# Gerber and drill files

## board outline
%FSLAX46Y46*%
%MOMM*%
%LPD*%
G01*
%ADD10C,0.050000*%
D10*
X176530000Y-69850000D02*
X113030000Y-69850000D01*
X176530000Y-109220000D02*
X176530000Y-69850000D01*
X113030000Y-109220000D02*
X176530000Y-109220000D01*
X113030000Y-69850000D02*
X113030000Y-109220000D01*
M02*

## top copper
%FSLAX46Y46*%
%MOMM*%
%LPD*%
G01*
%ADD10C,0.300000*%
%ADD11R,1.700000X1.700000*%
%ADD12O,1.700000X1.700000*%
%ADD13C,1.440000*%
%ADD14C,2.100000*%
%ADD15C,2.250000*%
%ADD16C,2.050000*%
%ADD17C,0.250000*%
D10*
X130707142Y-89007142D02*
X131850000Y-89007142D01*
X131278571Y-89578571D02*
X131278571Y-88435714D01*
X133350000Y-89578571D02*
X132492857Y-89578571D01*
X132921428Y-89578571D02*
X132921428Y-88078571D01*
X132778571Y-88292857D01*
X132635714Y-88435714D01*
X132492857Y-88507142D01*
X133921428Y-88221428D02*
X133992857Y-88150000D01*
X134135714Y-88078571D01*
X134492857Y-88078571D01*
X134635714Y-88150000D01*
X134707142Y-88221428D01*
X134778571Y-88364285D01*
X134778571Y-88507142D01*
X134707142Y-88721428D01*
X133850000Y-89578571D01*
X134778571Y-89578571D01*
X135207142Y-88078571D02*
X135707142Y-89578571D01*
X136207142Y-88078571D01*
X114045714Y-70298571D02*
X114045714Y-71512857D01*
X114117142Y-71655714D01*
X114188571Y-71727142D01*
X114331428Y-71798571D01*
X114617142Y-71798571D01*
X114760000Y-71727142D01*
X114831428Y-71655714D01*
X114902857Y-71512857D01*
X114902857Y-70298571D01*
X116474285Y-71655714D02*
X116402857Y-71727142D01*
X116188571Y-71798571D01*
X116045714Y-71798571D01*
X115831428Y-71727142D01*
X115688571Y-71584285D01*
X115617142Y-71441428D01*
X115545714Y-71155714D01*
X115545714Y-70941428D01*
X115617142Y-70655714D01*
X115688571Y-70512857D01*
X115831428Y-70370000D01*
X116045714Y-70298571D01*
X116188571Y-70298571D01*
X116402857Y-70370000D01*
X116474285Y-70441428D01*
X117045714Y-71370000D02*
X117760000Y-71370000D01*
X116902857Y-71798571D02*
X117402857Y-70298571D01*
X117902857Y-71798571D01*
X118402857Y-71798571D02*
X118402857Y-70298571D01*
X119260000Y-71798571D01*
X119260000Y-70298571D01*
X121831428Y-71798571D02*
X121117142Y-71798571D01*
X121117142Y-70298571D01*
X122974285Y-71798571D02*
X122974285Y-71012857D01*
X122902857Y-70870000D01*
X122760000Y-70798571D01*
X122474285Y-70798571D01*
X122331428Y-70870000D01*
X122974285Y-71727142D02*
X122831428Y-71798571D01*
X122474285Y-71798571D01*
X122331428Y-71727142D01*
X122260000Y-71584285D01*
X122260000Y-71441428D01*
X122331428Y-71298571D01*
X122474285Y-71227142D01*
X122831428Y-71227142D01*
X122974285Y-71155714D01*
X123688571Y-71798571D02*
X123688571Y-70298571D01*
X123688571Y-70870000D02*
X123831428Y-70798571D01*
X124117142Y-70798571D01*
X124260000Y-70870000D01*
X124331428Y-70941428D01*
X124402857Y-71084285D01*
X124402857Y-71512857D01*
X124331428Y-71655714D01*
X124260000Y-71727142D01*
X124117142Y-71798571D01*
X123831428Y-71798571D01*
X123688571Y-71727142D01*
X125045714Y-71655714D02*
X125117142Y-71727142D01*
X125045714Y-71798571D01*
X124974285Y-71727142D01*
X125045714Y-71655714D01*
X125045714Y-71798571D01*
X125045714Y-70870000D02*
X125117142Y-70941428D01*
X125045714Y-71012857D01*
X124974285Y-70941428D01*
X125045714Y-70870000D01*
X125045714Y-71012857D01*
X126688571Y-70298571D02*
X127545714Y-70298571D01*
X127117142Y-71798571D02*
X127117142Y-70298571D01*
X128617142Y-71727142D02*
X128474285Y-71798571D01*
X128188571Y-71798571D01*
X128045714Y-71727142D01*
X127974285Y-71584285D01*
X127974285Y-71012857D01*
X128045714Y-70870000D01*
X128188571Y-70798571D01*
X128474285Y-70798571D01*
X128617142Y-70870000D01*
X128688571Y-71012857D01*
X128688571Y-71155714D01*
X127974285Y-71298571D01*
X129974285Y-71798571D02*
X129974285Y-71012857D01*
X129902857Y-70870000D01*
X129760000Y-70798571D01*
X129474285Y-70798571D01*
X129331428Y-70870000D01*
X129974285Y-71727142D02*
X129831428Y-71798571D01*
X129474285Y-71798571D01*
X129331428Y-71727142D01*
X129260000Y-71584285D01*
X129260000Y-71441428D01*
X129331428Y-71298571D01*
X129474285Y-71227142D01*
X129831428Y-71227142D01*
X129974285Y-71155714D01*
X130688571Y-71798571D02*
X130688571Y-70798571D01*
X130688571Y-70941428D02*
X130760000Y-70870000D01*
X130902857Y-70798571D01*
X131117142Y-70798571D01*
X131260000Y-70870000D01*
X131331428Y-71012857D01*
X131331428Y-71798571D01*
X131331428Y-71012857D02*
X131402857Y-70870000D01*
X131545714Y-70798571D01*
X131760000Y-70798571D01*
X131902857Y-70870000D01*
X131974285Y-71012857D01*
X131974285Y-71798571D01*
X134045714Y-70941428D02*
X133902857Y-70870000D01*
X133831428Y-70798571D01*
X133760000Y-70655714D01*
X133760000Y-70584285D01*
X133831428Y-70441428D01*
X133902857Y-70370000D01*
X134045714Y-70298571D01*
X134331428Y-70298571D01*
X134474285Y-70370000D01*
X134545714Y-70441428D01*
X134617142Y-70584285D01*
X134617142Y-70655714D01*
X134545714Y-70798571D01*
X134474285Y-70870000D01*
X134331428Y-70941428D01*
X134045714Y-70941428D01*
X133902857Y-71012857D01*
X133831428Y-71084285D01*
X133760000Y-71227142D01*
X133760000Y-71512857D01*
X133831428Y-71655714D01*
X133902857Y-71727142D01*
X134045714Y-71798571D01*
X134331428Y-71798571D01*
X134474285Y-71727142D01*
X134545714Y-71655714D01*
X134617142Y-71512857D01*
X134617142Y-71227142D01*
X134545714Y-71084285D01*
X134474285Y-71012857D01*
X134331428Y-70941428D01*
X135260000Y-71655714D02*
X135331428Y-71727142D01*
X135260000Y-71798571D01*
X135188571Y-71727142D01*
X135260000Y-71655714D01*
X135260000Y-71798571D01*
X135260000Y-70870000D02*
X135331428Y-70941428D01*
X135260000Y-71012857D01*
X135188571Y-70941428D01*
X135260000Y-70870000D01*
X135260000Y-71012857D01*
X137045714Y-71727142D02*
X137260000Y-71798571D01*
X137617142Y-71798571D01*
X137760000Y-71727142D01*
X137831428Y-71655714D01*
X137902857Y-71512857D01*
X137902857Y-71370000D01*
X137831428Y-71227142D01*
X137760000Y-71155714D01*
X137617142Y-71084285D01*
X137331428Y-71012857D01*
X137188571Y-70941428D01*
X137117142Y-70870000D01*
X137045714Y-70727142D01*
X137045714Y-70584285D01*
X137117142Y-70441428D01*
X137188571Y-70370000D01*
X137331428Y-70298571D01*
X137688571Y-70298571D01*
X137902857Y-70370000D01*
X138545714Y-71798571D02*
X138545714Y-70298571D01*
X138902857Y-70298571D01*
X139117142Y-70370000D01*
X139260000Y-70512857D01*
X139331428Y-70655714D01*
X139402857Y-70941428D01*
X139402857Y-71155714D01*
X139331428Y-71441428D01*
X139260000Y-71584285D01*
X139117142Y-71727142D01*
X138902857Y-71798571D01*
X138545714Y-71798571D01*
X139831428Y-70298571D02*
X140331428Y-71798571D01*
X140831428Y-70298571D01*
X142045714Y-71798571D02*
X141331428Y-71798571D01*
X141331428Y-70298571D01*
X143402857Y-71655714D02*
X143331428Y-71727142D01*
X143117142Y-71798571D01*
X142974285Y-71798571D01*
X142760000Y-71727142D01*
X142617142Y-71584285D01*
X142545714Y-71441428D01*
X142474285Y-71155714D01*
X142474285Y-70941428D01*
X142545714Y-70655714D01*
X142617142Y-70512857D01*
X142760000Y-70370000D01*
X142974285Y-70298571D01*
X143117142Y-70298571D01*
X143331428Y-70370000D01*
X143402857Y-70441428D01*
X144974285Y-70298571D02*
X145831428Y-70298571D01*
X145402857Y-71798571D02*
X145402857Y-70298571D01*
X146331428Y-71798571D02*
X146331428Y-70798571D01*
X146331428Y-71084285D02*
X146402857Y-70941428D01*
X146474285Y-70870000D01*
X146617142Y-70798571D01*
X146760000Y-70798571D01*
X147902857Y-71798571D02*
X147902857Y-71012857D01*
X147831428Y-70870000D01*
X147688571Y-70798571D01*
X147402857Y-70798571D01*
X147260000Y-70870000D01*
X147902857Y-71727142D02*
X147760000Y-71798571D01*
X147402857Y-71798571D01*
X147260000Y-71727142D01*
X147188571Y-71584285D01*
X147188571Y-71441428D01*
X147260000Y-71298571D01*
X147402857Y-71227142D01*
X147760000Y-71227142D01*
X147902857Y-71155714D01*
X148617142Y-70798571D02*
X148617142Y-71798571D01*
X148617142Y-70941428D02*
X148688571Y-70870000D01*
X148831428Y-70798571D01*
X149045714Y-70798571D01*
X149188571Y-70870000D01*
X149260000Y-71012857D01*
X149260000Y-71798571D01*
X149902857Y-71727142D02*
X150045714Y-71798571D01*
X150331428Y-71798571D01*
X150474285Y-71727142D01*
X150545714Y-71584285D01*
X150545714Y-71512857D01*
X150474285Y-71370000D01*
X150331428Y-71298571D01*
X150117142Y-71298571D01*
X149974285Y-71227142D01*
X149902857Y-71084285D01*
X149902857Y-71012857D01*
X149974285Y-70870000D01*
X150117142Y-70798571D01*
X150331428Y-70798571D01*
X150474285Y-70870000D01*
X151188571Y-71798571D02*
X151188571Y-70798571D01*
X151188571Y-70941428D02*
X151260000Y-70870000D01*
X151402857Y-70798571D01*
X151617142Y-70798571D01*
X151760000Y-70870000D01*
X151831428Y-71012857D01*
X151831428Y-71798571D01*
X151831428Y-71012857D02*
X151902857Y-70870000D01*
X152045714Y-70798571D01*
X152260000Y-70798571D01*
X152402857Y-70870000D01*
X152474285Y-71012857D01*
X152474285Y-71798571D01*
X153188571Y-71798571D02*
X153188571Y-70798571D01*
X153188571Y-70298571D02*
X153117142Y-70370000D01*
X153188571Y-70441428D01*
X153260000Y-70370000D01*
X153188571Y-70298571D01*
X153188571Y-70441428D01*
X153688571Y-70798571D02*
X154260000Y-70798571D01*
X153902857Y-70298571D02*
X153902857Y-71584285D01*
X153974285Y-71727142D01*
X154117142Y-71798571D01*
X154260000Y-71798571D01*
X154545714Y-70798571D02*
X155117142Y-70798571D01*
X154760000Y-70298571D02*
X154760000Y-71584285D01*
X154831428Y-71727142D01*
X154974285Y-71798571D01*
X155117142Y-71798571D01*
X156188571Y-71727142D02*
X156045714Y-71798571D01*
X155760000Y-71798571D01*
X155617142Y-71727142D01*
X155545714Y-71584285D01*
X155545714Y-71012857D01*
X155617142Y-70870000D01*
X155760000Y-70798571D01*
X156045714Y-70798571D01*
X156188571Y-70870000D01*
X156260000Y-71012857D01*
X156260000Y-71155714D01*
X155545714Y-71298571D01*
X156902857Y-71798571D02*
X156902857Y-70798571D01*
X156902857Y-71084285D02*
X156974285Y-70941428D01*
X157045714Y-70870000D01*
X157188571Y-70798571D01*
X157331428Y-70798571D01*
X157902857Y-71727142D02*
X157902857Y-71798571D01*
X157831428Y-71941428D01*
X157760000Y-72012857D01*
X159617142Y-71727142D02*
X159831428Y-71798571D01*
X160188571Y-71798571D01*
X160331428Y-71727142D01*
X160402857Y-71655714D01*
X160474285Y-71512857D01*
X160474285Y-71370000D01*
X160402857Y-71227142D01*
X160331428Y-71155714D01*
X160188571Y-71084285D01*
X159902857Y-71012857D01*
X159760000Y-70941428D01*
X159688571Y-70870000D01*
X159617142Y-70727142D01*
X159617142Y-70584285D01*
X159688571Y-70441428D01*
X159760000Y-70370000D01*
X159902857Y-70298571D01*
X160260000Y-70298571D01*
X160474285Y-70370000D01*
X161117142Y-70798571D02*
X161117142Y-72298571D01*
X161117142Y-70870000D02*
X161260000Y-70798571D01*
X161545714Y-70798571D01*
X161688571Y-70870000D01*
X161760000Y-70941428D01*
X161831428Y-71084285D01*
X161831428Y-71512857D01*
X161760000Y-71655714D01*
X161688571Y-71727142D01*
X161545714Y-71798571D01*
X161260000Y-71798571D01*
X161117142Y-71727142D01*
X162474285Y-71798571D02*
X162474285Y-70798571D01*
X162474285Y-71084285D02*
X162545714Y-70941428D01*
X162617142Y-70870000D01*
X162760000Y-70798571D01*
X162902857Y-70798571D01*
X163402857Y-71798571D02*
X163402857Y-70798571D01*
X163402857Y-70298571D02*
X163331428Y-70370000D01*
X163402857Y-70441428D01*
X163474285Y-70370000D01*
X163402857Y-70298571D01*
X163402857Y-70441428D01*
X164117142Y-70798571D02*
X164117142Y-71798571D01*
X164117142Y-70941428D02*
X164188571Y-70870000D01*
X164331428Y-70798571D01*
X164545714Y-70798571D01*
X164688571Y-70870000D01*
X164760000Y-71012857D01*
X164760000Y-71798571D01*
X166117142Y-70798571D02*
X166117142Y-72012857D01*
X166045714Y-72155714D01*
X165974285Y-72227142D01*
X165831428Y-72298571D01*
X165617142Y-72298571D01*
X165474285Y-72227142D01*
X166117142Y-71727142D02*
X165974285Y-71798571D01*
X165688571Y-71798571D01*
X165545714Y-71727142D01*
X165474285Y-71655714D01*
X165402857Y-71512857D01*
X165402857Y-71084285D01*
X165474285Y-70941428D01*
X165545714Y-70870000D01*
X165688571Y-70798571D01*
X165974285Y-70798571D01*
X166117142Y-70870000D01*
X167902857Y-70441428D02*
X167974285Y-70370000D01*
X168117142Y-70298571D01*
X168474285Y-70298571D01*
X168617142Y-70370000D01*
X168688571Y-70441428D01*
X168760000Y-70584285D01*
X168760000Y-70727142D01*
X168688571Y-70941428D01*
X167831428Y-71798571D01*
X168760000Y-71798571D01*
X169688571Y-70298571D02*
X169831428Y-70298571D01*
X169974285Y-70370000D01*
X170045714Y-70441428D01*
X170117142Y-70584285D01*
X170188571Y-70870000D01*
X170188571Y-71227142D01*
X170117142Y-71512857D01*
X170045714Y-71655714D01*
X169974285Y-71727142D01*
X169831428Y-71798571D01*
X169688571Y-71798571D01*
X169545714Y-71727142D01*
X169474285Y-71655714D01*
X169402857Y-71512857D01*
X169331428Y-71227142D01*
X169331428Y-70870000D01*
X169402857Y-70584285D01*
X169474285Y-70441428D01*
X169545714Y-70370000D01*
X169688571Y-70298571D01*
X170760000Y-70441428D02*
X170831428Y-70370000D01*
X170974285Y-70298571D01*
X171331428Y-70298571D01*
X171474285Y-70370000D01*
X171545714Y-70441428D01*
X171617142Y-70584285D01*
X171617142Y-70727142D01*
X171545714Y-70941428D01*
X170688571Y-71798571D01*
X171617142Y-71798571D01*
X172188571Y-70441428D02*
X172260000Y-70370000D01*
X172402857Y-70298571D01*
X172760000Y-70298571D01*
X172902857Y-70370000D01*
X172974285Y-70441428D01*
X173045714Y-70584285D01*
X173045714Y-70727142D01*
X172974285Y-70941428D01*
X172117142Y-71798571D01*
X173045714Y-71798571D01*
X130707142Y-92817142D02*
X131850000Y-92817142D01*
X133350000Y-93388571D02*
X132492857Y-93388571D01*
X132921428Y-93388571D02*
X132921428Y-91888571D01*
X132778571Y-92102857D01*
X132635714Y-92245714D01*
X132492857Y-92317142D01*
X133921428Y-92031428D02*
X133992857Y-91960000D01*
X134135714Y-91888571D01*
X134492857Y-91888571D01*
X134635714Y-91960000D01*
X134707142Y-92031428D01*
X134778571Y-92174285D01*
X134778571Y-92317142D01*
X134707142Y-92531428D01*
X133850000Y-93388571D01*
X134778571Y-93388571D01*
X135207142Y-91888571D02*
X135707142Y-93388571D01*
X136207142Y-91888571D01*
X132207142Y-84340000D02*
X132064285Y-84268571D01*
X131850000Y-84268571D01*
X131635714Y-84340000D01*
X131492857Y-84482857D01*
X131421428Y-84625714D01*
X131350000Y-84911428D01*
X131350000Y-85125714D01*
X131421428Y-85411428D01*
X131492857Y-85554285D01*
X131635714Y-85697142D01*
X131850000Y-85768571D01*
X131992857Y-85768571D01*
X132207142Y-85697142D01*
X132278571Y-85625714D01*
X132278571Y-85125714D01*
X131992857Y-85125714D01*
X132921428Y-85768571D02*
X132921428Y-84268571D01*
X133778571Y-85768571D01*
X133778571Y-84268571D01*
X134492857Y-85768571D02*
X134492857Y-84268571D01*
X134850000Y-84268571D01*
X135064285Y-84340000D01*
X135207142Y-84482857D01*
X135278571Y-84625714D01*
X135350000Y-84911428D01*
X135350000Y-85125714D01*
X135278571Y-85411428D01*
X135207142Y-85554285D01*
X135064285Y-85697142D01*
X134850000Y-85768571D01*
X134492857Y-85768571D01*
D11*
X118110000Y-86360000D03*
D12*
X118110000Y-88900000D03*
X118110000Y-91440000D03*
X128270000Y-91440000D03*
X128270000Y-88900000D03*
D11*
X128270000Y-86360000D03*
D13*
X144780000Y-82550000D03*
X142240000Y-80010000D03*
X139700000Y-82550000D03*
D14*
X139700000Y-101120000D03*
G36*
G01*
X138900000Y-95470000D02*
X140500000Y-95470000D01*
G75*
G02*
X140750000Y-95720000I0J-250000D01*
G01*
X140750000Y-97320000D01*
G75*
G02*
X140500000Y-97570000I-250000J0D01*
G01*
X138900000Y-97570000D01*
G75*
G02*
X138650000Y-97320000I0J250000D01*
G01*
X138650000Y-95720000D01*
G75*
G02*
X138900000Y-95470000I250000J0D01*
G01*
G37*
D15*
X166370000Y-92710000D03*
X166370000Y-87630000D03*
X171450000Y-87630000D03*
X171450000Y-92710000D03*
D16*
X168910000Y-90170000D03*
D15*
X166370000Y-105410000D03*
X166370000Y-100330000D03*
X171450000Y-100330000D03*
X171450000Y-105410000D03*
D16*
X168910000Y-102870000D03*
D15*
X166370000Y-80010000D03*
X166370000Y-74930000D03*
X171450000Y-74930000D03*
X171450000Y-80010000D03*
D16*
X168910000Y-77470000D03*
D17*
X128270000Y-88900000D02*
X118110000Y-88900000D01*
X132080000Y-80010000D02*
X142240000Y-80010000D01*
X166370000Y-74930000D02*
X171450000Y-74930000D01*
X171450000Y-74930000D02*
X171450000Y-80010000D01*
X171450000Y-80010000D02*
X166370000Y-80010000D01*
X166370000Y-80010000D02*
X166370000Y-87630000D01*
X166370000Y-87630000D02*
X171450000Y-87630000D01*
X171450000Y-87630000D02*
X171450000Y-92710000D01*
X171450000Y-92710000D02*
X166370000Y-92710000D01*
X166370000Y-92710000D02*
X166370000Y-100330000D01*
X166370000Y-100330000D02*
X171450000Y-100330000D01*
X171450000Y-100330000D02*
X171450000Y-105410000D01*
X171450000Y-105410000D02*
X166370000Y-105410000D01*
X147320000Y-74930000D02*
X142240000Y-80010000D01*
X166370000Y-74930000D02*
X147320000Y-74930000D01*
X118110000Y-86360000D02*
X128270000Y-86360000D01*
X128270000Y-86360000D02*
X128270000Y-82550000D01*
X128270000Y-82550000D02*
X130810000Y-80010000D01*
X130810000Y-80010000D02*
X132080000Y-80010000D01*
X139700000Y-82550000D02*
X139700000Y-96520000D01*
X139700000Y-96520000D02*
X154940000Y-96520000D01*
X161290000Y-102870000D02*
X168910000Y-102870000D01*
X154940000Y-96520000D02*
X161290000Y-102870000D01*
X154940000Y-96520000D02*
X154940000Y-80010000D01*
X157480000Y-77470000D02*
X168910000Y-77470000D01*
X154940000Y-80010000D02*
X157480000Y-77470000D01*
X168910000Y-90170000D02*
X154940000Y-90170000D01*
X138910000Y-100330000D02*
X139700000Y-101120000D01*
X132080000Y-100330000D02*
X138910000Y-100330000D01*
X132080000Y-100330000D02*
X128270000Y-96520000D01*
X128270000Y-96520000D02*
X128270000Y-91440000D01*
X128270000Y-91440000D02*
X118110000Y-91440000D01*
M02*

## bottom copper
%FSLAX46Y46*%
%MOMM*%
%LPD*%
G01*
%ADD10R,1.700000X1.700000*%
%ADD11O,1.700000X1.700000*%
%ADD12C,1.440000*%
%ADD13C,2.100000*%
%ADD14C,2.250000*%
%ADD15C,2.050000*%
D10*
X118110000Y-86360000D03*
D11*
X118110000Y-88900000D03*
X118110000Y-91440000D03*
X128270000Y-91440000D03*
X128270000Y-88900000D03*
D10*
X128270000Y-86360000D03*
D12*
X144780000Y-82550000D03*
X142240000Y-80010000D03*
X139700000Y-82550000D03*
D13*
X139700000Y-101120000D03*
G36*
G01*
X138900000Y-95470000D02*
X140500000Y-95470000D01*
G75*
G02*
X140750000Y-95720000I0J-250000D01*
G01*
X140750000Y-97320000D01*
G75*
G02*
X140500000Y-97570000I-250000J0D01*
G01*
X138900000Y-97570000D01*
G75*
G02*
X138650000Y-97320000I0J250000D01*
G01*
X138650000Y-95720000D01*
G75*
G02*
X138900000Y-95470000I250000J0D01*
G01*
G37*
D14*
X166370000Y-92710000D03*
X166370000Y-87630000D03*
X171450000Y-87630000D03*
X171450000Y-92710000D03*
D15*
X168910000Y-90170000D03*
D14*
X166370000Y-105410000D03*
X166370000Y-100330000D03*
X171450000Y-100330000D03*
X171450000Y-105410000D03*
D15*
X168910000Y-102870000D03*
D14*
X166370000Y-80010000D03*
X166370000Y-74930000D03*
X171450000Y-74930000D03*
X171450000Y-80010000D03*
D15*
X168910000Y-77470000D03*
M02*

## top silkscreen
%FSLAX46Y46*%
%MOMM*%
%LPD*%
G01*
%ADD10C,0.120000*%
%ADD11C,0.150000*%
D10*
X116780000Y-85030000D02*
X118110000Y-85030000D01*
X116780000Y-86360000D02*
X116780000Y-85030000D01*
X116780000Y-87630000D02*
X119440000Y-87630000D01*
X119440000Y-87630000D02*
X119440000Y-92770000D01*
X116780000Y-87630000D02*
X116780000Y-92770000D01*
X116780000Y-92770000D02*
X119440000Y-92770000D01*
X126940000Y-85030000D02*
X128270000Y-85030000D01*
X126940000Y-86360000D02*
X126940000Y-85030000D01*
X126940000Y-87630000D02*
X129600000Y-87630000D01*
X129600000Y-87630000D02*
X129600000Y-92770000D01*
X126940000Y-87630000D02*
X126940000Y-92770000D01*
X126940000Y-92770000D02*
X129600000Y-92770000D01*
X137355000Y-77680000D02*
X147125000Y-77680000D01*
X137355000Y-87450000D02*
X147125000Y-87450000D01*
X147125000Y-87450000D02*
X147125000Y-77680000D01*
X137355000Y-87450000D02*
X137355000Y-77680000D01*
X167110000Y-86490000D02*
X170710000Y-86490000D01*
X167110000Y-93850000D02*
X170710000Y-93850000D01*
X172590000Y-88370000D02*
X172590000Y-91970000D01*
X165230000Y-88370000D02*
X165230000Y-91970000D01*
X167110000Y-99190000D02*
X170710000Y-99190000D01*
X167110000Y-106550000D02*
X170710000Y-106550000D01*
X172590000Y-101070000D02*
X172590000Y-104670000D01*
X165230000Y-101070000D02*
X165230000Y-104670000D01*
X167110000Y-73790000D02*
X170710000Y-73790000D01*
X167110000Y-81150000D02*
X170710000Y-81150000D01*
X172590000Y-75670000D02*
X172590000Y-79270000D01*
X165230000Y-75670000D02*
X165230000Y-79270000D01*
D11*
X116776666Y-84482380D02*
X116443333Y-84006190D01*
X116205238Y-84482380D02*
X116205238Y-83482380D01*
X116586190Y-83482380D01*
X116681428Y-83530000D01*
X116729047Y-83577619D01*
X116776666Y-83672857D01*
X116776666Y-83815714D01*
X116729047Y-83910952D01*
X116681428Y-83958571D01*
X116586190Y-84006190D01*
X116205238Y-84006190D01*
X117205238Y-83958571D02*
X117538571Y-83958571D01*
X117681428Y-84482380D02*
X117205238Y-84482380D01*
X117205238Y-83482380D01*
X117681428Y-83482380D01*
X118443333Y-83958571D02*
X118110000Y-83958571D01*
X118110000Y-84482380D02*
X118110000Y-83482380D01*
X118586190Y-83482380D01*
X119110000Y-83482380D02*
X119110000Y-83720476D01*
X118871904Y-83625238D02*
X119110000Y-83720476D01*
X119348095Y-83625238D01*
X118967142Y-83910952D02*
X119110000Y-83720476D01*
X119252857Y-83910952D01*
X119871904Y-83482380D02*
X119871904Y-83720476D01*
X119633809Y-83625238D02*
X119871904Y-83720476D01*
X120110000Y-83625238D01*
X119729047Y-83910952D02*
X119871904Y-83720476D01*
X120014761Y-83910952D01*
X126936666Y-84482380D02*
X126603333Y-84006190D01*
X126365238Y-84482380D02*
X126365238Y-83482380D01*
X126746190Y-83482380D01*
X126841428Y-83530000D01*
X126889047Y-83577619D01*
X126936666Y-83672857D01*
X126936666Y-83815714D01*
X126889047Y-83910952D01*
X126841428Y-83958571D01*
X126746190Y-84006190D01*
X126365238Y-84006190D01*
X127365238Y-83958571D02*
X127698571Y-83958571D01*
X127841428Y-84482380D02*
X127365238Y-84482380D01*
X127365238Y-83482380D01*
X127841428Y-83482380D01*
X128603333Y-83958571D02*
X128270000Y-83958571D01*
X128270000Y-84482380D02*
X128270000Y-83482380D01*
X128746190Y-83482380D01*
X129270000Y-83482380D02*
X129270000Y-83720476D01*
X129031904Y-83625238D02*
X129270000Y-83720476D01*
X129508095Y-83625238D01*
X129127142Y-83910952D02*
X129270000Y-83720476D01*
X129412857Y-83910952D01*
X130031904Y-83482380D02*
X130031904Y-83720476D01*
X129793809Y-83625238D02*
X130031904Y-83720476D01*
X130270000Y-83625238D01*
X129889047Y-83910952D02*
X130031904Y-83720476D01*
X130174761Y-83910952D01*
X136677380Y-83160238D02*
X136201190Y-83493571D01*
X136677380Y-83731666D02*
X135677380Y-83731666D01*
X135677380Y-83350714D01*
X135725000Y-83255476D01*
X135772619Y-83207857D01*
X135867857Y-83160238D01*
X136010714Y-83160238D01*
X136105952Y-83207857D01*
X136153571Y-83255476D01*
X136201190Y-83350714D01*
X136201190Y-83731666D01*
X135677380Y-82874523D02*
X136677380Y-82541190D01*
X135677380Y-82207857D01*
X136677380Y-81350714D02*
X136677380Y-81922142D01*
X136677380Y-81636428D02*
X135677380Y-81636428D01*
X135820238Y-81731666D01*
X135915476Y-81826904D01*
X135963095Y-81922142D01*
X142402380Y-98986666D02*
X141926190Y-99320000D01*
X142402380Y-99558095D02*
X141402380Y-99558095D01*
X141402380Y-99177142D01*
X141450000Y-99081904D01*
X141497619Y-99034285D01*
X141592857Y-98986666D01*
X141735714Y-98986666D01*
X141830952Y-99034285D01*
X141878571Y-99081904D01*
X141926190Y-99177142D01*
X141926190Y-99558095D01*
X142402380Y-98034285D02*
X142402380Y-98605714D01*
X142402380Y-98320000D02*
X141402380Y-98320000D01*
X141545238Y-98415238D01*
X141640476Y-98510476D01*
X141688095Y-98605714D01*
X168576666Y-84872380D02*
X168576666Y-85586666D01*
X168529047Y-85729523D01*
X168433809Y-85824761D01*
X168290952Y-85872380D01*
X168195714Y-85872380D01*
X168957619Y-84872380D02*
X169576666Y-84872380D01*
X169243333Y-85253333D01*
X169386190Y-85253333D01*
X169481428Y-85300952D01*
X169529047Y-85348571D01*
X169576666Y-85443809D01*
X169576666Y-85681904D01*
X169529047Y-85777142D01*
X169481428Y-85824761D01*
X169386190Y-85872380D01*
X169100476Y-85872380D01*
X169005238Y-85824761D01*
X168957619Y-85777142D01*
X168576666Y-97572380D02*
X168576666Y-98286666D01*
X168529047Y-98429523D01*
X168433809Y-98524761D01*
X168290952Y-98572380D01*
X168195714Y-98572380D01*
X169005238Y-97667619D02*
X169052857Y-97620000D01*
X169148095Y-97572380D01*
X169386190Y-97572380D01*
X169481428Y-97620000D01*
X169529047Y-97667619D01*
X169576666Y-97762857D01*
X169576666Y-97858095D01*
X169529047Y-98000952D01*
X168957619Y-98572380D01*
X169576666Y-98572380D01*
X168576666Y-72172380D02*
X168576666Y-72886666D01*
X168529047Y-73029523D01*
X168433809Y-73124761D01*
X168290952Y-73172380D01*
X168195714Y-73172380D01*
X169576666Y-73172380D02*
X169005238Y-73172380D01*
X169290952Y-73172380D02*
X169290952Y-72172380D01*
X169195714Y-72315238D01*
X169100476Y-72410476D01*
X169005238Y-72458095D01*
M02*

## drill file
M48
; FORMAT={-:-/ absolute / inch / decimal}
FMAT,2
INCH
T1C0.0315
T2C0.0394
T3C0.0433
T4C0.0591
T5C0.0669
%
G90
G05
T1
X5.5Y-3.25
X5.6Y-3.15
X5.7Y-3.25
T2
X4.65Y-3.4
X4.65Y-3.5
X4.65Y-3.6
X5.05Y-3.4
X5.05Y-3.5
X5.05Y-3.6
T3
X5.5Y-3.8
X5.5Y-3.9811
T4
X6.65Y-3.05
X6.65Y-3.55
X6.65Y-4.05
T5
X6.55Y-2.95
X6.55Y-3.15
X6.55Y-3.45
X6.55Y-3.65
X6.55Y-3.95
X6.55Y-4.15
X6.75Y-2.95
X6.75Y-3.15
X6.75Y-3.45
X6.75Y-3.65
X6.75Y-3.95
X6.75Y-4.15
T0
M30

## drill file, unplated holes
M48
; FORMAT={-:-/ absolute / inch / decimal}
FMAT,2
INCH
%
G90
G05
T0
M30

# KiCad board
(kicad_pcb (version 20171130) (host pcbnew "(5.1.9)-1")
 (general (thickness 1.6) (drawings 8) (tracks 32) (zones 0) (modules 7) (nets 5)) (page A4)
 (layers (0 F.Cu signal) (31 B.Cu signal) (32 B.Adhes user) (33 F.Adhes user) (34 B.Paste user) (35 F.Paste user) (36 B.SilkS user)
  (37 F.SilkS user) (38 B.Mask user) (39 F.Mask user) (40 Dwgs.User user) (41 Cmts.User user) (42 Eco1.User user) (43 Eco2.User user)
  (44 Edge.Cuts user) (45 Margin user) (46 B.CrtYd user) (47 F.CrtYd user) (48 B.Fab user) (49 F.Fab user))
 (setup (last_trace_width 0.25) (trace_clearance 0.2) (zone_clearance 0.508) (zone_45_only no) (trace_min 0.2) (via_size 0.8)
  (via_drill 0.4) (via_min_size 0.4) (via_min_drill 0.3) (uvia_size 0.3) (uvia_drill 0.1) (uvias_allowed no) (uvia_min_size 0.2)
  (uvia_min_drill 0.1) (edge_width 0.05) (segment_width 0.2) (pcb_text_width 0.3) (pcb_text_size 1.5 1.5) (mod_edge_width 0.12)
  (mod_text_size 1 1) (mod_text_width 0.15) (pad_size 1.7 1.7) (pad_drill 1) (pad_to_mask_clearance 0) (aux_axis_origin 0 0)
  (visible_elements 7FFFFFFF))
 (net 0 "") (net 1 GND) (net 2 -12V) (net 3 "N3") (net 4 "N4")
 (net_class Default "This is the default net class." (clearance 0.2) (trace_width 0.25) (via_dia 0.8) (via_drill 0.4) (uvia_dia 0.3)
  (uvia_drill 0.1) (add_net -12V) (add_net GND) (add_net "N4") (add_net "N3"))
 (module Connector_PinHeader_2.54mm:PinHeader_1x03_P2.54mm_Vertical (layer F.Cu) (at 118.11 86.36)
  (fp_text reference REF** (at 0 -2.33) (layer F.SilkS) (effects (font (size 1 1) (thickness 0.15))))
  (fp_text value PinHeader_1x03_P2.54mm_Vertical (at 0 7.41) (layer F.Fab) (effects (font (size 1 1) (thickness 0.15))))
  (fp_line (start -1.33 -1.33) (end 0 -1.33) (layer F.SilkS) (width 0.12))
  (fp_line (start -1.33 0) (end -1.33 -1.33) (layer F.SilkS) (width 0.12))
  (fp_line (start -1.33 1.27) (end 1.33 1.27) (layer F.SilkS) (width 0.12))
  (fp_line (start 1.33 1.27) (end 1.33 6.41) (layer F.SilkS) (width 0.12))
  (fp_line (start -1.33 1.27) (end -1.33 6.41) (layer F.SilkS) (width 0.12))
  (fp_line (start -1.33 6.41) (end 1.33 6.41) (layer F.SilkS) (width 0.12))
  (pad 1 thru_hole rect (at 0 0) (size 1.7 1.7) (drill 1) (layers *.Cu *.Mask) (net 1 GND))
  (pad 2 thru_hole oval (at 0 2.54) (size 1.7 1.7) (drill 1) (layers *.Cu *.Mask))
  (pad 3 thru_hole oval (at 0 5.08) (size 1.7 1.7) (drill 1) (layers *.Cu *.Mask) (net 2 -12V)))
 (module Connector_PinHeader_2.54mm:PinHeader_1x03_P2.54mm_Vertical (layer F.Cu) (at 128.27 86.36)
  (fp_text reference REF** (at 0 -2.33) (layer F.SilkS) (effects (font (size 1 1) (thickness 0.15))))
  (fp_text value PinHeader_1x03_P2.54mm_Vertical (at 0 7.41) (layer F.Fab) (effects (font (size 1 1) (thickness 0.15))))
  (fp_line (start -1.33 -1.33) (end 0 -1.33) (layer F.SilkS) (width 0.12))
  (fp_line (start -1.33 0) (end -1.33 -1.33) (layer F.SilkS) (width 0.12))
  (fp_line (start -1.33 1.27) (end 1.33 1.27) (layer F.SilkS) (width 0.12))
  (fp_line (start 1.33 1.27) (end 1.33 6.41) (layer F.SilkS) (width 0.12))
  (fp_line (start -1.33 1.27) (end -1.33 6.41) (layer F.SilkS) (width 0.12))
  (fp_line (start -1.33 6.41) (end 1.33 6.41) (layer F.SilkS) (width 0.12))
  (pad 3 thru_hole oval (at 0 5.08) (size 1.7 1.7) (drill 1) (layers *.Cu *.Mask) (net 2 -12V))
  (pad 2 thru_hole oval (at 0 2.54) (size 1.7 1.7) (drill 1) (layers *.Cu *.Mask))
  (pad 1 thru_hole rect (at 0 0) (size 1.7 1.7) (drill 1) (layers *.Cu *.Mask) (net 1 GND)))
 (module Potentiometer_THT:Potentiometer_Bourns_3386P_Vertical (layer F.Cu) (at 144.78 82.55 90)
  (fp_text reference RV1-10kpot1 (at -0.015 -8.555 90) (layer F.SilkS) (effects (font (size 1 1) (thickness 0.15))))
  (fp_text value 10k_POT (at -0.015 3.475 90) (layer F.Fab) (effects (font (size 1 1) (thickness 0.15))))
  (fp_line (start 4.87 -7.425) (end 4.87 2.345) (layer F.SilkS) (width 0.12))
  (fp_line (start -4.9 -7.425) (end -4.9 2.345) (layer F.SilkS) (width 0.12))
  (fp_line (start -4.9 2.345) (end 4.87 2.345) (layer F.SilkS) (width 0.12))
  (fp_line (start -4.9 -7.425) (end 4.87 -7.425) (layer F.SilkS) (width 0.12))
  (pad 1 thru_hole circle (at 0 0 90) (size 1.44 1.44) (drill 0.8) (layers *.Cu *.Mask) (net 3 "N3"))
  (pad 2 thru_hole circle (at 2.54 -2.54 90) (size 1.44 1.44) (drill 0.8) (layers *.Cu *.Mask) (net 1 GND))
  (pad 3 thru_hole circle (at 0 -5.08 90) (size 1.44 1.44) (drill 0.8) (layers *.Cu *.Mask) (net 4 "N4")))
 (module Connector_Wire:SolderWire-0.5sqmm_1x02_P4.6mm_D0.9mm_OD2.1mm (layer F.Cu) (at 139.7 96.52 270)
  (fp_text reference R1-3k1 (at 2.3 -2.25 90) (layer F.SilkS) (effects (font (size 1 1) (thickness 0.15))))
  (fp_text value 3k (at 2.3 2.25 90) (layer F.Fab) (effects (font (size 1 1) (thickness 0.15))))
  (pad 2 thru_hole circle (at 4.6 0 270) (size 2.1 2.1) (drill 1.1) (layers *.Cu *.Mask) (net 2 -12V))
  (pad 1 thru_hole roundrect (at 0 0 270) (size 2.1 2.1) (drill 1.1) (layers *.Cu *.Mask) (roundrect_rratio 0.119047619047619) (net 4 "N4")))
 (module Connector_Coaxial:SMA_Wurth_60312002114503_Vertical (layer F.Cu) (at 168.91 90.17)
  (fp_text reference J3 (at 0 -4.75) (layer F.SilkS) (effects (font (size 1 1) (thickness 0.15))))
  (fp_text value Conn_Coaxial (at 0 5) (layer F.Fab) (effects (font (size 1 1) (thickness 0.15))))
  (fp_line (start -1.8 -3.68) (end 1.8 -3.68) (layer F.SilkS) (width 0.12))
  (fp_line (start -1.8 3.68) (end 1.8 3.68) (layer F.SilkS) (width 0.12))
  (fp_line (start 3.68 -1.8) (end 3.68 1.8) (layer F.SilkS) (width 0.12))
  (fp_line (start -3.68 -1.8) (end -3.68 1.8) (layer F.SilkS) (width 0.12))
  (pad 2 thru_hole circle (at -2.54 2.54) (size 2.25 2.25) (drill 1.7) (layers *.Cu *.Mask) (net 1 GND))
  (pad 2 thru_hole circle (at -2.54 -2.54) (size 2.25 2.25) (drill 1.7) (layers *.Cu *.Mask) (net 1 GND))
  (pad 2 thru_hole circle (at 2.54 -2.54) (size 2.25 2.25) (drill 1.7) (layers *.Cu *.Mask) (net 1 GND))
  (pad 2 thru_hole circle (at 2.54 2.54) (size 2.25 2.25) (drill 1.7) (layers *.Cu *.Mask) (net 1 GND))
  (pad 1 thru_hole circle (at 0 0) (size 2.05 2.05) (drill 1.5) (layers *.Cu *.Mask) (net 4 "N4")))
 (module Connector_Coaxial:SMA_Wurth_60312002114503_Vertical (layer F.Cu) (at 168.91 102.87)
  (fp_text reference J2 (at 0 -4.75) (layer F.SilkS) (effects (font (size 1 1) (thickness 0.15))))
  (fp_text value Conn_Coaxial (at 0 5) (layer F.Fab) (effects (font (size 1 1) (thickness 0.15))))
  (fp_line (start -1.8 -3.68) (end 1.8 -3.68) (layer F.SilkS) (width 0.12))
  (fp_line (start -1.8 3.68) (end 1.8 3.68) (layer F.SilkS) (width 0.12))
  (fp_line (start 3.68 -1.8) (end 3.68 1.8) (layer F.SilkS) (width 0.12))
  (fp_line (start -3.68 -1.8) (end -3.68 1.8) (layer F.SilkS) (width 0.12))
  (pad 2 thru_hole circle (at -2.54 2.54) (size 2.25 2.25) (drill 1.7) (layers *.Cu *.Mask) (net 1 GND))
  (pad 2 thru_hole circle (at -2.54 -2.54) (size 2.25 2.25) (drill 1.7) (layers *.Cu *.Mask) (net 1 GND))
  (pad 2 thru_hole circle (at 2.54 -2.54) (size 2.25 2.25) (drill 1.7) (layers *.Cu *.Mask) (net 1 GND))
  (pad 2 thru_hole circle (at 2.54 2.54) (size 2.25 2.25) (drill 1.7) (layers *.Cu *.Mask) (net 1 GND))
  (pad 1 thru_hole circle (at 0 0) (size 2.05 2.05) (drill 1.5) (layers *.Cu *.Mask) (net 4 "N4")))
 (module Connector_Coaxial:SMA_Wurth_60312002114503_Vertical (layer F.Cu) (at 168.91 77.47)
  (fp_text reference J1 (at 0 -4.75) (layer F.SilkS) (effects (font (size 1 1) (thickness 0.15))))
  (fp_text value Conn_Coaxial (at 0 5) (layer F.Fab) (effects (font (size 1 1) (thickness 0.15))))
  (fp_line (start -1.8 -3.68) (end 1.8 -3.68) (layer F.SilkS) (width 0.12))
  (fp_line (start -1.8 3.68) (end 1.8 3.68) (layer F.SilkS) (width 0.12))
  (fp_line (start 3.68 -1.8) (end 3.68 1.8) (layer F.SilkS) (width 0.12))
  (fp_line (start -3.68 -1.8) (end -3.68 1.8) (layer F.SilkS) (width 0.12))
  (pad 2 thru_hole circle (at -2.54 2.54) (size 2.25 2.25) (drill 1.7) (layers *.Cu *.Mask) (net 1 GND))
  (pad 2 thru_hole circle (at -2.54 -2.54) (size 2.25 2.25) (drill 1.7) (layers *.Cu *.Mask) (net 1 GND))
  (pad 2 thru_hole circle (at 2.54 -2.54) (size 2.25 2.25) (drill 1.7) (layers *.Cu *.Mask) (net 1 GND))
  (pad 2 thru_hole circle (at 2.54 2.54) (size 2.25 2.25) (drill 1.7) (layers *.Cu *.Mask) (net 1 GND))
  (pad 1 thru_hole circle (at 0 0) (size 2.05 2.05) (drill 1.5) (layers *.Cu *.Mask) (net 4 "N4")))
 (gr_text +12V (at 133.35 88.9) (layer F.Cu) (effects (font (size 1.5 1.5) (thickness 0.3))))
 (gr_line (start 176.53 69.85) (end 113.03 69.85) (layer Edge.Cuts) (width 0.05))
 (gr_line (start 176.53 109.22) (end 176.53 69.85) (layer Edge.Cuts) (width 0.05))
 (gr_line (start 113.03 109.22) (end 176.53 109.22) (layer Edge.Cuts) (width 0.05))
 (gr_line (start 113.03 69.85) (end 113.03 109.22) (layer Edge.Cuts) (width 0.05))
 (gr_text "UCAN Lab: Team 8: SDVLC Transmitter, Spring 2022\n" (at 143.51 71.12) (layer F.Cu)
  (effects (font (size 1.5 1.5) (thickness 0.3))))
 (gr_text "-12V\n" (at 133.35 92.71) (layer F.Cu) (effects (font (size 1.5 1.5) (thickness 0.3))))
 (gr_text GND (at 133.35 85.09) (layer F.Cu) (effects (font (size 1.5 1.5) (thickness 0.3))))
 (segment (start 128.27 88.9) (end 118.11 88.9) (width 0.25) (layer F.Cu) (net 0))
 (segment (start 132.08 80.01) (end 142.24 80.01) (width 0.25) (layer F.Cu) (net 1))
 (segment (start 166.37 74.93) (end 171.45 74.93) (width 0.25) (layer F.Cu) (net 1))
 (segment (start 171.45 74.93) (end 171.45 80.01) (width 0.25) (layer F.Cu) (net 1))
 (segment (start 171.45 80.01) (end 166.37 80.01) (width 0.25) (layer F.Cu) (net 1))
 (segment (start 166.37 80.01) (end 166.37 87.63) (width 0.25) (layer F.Cu) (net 1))
 (segment (start 166.37 87.63) (end 171.45 87.63) (width 0.25) (layer F.Cu) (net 1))
 (segment (start 171.45 87.63) (end 171.45 92.71) (width 0.25) (layer F.Cu) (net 1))
 (segment (start 171.45 92.71) (end 166.37 92.71) (width 0.25) (layer F.Cu) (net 1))
 (segment (start 166.37 92.71) (end 166.37 100.33) (width 0.25) (layer F.Cu) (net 1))
 (segment (start 166.37 100.33) (end 171.45 100.33) (width 0.25) (layer F.Cu) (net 1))
 (segment (start 171.45 100.33) (end 171.45 105.41) (width 0.25) (layer F.Cu) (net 1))
 (segment (start 171.45 105.41) (end 166.37 105.41) (width 0.25) (layer F.Cu) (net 1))
 (segment (start 147.32 74.93) (end 142.24 80.01) (width 0.25) (layer F.Cu) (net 1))
 (segment (start 166.37 74.93) (end 147.32 74.93) (width 0.25) (layer F.Cu) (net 1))
 (segment (start 118.11 86.36) (end 128.27 86.36) (width 0.25) (layer F.Cu) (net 1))
 (segment (start 128.27 86.36) (end 128.27 82.55) (width 0.25) (layer F.Cu) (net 1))
 (segment (start 128.27 82.55) (end 130.81 80.01) (width 0.25) (layer F.Cu) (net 1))
 (segment (start 130.81 80.01) (end 132.08 80.01) (width 0.25) (layer F.Cu) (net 1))
 (segment (start 139.7 82.55) (end 139.7 96.52) (width 0.25) (layer F.Cu) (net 4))
 (segment (start 139.7 96.52) (end 154.94 96.52) (width 0.25) (layer F.Cu) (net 4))
 (segment (start 161.29 102.87) (end 168.91 102.87) (width 0.25) (layer F.Cu) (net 4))
 (segment (start 154.94 96.52) (end 161.29 102.87) (width 0.25) (layer F.Cu) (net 4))
 (segment (start 154.94 96.52) (end 154.94 80.01) (width 0.25) (layer F.Cu) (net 4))
 (segment (start 157.48 77.47) (end 168.91 77.47) (width 0.25) (layer F.Cu) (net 4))
 (segment (start 154.94 80.01) (end 157.48 77.47) (width 0.25) (layer F.Cu) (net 4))
 (segment (start 168.91 90.17) (end 154.94 90.17) (width 0.25) (layer F.Cu) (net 4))
 (segment (start 138.91 100.33) (end 139.7 101.12) (width 0.25) (layer F.Cu) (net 2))
 (segment (start 132.08 100.33) (end 138.91 100.33) (width 0.25) (layer F.Cu) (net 2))
 (segment (start 132.08 100.33) (end 128.27 96.52) (width 0.25) (layer F.Cu) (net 2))
 (segment (start 128.27 96.52) (end 128.27 91.44) (width 0.25) (layer F.Cu) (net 2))
 (segment (start 128.27 91.44) (end 118.11 91.44) (width 0.25) (layer F.Cu) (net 2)))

